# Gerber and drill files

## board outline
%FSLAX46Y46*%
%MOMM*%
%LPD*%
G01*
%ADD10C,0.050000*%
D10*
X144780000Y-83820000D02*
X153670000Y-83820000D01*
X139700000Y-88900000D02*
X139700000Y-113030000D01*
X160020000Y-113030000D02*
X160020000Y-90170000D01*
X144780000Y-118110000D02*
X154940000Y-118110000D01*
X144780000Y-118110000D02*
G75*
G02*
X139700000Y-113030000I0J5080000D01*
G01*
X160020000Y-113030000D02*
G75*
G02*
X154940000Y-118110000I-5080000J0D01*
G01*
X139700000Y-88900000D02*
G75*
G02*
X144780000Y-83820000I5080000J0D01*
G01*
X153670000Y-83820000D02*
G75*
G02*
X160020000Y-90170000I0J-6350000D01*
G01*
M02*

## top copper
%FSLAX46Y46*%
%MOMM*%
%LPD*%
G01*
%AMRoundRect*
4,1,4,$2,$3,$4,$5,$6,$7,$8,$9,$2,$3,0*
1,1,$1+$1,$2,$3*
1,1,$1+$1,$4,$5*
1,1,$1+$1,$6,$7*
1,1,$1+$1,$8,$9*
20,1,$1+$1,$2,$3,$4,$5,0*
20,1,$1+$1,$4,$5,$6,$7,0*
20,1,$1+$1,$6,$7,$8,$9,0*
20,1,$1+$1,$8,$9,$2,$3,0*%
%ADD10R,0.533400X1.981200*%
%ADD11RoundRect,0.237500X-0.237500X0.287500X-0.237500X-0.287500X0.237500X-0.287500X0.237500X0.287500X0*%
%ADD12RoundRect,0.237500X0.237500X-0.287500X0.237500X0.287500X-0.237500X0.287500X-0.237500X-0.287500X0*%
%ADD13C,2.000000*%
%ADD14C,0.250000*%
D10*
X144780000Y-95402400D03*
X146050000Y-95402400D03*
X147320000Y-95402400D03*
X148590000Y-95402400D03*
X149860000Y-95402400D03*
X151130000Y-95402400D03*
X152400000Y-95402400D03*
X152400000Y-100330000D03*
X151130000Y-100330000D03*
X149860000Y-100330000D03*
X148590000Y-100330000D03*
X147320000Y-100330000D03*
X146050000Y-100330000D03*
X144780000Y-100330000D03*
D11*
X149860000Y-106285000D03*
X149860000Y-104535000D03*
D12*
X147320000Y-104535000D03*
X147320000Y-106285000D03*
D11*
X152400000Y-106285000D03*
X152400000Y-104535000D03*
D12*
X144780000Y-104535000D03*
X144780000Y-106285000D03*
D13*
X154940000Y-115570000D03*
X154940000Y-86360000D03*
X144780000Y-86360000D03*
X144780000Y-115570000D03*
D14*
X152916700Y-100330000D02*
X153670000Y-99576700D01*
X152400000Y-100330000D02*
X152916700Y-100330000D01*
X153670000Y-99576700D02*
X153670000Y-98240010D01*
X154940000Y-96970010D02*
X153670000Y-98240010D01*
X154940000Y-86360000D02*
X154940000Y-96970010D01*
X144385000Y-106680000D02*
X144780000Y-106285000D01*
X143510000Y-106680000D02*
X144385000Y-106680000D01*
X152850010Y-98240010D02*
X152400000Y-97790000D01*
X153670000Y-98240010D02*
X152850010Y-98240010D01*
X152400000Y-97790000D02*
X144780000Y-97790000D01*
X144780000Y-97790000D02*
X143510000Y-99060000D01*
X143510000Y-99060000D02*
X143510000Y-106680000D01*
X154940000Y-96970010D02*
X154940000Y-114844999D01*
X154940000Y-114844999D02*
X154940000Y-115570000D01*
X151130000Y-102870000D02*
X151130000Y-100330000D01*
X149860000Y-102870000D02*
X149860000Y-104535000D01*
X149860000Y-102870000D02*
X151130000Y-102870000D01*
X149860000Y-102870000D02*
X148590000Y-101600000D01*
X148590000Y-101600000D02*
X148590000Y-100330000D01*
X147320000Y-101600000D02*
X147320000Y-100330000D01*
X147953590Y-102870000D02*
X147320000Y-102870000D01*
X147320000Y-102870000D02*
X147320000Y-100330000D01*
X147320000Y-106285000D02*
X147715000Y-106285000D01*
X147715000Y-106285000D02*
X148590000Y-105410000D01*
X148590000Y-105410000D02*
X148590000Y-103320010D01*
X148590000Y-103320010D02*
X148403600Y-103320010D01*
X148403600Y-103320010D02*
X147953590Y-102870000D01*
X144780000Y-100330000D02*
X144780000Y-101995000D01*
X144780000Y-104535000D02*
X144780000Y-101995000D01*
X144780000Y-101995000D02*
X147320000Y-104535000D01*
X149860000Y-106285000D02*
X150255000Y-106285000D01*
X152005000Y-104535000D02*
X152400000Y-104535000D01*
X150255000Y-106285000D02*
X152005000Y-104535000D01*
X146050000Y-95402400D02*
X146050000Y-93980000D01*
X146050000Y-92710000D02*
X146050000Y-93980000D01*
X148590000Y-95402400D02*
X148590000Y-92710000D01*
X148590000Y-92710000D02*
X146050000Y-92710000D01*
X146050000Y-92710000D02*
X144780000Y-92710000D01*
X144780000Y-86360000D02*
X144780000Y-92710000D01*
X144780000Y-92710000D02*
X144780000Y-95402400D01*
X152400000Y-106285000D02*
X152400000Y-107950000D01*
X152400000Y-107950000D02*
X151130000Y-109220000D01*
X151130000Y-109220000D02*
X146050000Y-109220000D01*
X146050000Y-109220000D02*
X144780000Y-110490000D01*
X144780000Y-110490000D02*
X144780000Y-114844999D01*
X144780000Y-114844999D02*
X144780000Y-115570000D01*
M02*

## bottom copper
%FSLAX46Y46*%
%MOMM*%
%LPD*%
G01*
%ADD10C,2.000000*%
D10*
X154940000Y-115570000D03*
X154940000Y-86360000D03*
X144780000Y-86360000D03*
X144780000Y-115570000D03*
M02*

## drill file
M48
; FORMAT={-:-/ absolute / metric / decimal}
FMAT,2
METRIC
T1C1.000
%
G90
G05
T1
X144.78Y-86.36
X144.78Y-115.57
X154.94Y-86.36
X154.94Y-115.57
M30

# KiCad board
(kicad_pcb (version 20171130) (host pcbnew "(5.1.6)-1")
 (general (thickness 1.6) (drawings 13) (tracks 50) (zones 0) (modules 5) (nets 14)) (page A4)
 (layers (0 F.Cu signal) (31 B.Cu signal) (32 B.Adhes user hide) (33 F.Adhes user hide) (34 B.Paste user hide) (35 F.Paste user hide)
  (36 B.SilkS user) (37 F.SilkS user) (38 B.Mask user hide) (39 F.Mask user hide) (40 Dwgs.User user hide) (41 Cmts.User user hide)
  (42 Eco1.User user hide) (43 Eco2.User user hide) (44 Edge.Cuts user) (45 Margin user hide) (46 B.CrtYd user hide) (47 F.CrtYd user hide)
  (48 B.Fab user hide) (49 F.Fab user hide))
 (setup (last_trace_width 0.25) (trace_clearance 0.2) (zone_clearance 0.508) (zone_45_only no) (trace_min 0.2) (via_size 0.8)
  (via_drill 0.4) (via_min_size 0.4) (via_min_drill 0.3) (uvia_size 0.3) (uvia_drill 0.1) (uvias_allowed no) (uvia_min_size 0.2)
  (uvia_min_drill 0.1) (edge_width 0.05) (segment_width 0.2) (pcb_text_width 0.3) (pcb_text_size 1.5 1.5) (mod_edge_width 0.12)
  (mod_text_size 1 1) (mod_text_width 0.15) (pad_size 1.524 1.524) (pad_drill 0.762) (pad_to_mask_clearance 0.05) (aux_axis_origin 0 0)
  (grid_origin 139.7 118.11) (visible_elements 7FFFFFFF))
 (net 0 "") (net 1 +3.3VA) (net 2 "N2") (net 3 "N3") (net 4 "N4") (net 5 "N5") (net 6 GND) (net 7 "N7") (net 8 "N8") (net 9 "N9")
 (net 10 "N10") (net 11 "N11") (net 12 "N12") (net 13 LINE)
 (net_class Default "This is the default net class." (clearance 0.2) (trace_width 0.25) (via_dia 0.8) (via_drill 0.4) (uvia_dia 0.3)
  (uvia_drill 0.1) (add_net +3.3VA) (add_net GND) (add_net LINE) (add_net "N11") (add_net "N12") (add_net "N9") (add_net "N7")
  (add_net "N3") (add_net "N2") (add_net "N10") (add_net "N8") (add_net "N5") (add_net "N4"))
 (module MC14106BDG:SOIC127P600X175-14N (layer F.Cu) (at 148.59 97.8662 90)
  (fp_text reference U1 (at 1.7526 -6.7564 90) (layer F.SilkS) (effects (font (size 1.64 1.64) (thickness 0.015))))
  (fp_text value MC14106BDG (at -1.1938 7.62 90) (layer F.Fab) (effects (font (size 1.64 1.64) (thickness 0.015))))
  (pad 14 smd rect (at 2.4638 -3.81 90) (size 1.9812 0.5334) (layers F.Cu F.Paste F.Mask) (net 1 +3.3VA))
  (pad 13 smd rect (at 2.4638 -2.54 90) (size 1.9812 0.5334) (layers F.Cu F.Paste F.Mask) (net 1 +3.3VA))
  (pad 12 smd rect (at 2.4638 -1.27 90) (size 1.9812 0.5334) (layers F.Cu F.Paste F.Mask) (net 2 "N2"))
  (pad 11 smd rect (at 2.4638 0 90) (size 1.9812 0.5334) (layers F.Cu F.Paste F.Mask) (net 1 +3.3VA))
  (pad 10 smd rect (at 2.4638 1.27 90) (size 1.9812 0.5334) (layers F.Cu F.Paste F.Mask) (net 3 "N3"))
  (pad 9 smd rect (at 2.4638 2.54 90) (size 1.9812 0.5334) (layers F.Cu F.Paste F.Mask) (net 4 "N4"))
  (pad 8 smd rect (at 2.4638 3.81 90) (size 1.9812 0.5334) (layers F.Cu F.Paste F.Mask) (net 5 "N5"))
  (pad 7 smd rect (at -2.4638 3.81 90) (size 1.9812 0.5334) (layers F.Cu F.Paste F.Mask) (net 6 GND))
  (pad 6 smd rect (at -2.4638 2.54 90) (size 1.9812 0.5334) (layers F.Cu F.Paste F.Mask) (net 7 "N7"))
  (pad 5 smd rect (at -2.4638 1.27 90) (size 1.9812 0.5334) (layers F.Cu F.Paste F.Mask) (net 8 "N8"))
  (pad 4 smd rect (at -2.4638 0 90) (size 1.9812 0.5334) (layers F.Cu F.Paste F.Mask) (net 7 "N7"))
  (pad 3 smd rect (at -2.4638 -1.27 90) (size 1.9812 0.5334) (layers F.Cu F.Paste F.Mask) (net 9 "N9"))
  (pad 2 smd rect (at -2.4638 -2.54 90) (size 1.9812 0.5334) (layers F.Cu F.Paste F.Mask) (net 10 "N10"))
  (pad 1 smd rect (at -2.4638 -3.81 90) (size 1.9812 0.5334) (layers F.Cu F.Paste F.Mask) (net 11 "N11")))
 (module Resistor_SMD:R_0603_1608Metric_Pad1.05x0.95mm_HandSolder (layer F.Cu) (at 149.86 105.41 270)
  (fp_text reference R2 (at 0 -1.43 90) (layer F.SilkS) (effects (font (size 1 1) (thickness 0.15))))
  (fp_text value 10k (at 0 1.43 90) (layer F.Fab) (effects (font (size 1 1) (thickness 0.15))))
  (pad 2 smd roundrect (at 0.875 0 270) (size 1.05 0.95) (layers F.Cu F.Paste F.Mask) (roundrect_rratio 0.25) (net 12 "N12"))
  (pad 1 smd roundrect (at -0.875 0 270) (size 1.05 0.95) (layers F.Cu F.Paste F.Mask) (roundrect_rratio 0.25) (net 7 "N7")))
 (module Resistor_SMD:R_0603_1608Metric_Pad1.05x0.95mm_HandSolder (layer F.Cu) (at 147.32 105.41 90)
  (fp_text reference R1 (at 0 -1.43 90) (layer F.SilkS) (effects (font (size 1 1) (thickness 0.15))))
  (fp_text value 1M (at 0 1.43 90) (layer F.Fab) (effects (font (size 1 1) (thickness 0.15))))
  (pad 2 smd roundrect (at 0.875 0 90) (size 1.05 0.95) (layers F.Cu F.Paste F.Mask) (roundrect_rratio 0.25) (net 11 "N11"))
  (pad 1 smd roundrect (at -0.875 0 90) (size 1.05 0.95) (layers F.Cu F.Paste F.Mask) (roundrect_rratio 0.25) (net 9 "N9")))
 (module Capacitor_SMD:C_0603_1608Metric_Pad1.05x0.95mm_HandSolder (layer F.Cu) (at 152.4 105.41 270)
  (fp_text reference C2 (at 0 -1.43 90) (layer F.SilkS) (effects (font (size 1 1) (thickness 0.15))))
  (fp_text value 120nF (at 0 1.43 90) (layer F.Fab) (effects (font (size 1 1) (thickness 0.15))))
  (pad 2 smd roundrect (at 0.875 0 270) (size 1.05 0.95) (layers F.Cu F.Paste F.Mask) (roundrect_rratio 0.25) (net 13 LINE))
  (pad 1 smd roundrect (at -0.875 0 270) (size 1.05 0.95) (layers F.Cu F.Paste F.Mask) (roundrect_rratio 0.25) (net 12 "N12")))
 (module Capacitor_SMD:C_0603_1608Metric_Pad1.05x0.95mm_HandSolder (layer F.Cu) (at 144.78 105.41 90)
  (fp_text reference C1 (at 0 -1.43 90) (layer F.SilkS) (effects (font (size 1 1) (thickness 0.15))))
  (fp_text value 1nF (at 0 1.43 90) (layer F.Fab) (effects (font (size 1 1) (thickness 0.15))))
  (pad 2 smd roundrect (at 0.875 0 90) (size 1.05 0.95) (layers F.Cu F.Paste F.Mask) (roundrect_rratio 0.25) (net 11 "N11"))
  (pad 1 smd roundrect (at -0.875 0 90) (size 1.05 0.95) (layers F.Cu F.Paste F.Mask) (roundrect_rratio 0.25) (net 6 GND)))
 (gr_line (start 144.78 83.82) (end 153.67 83.82) (layer Edge.Cuts) (width 0.05))
 (gr_line (start 139.7 88.9) (end 139.7 113.03) (layer Edge.Cuts) (width 0.05))
 (gr_line (start 160.02 113.03) (end 160.02 90.17) (layer Edge.Cuts) (width 0.05))
 (gr_line (start 144.78 118.11) (end 154.94 118.11) (layer Edge.Cuts) (width 0.05))
 (gr_arc (start 144.78 113.03) (end 139.7 113.03) (angle -90) (layer Edge.Cuts) (width 0.05))
 (gr_arc (start 154.94 113.03) (end 154.94 118.11) (angle -90) (layer Edge.Cuts) (width 0.05))
 (gr_arc (start 144.78 88.9) (end 144.78 83.82) (angle -90) (layer Edge.Cuts) (width 0.05))
 (gr_arc (start 153.67 90.17) (end 160.02 90.17) (angle -90) (layer Edge.Cuts) (width 0.05))
 (via (at 154.94 115.57) (size 2) (drill 1) (layers F.Cu B.Cu) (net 6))
 (via (at 154.94 86.36) (size 2) (drill 1) (layers F.Cu B.Cu) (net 6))
 (segment (start 152.9167 100.33) (end 153.67 99.5767) (width 0.25) (layer F.Cu) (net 6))
 (segment (start 152.4 100.33) (end 152.9167 100.33) (width 0.25) (layer F.Cu) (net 6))
 (segment (start 153.67 99.5767) (end 153.67 98.24001) (width 0.25) (layer F.Cu) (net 6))
 (segment (start 154.94 96.97001) (end 153.67 98.24001) (width 0.25) (layer F.Cu) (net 6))
 (segment (start 154.94 86.36) (end 154.94 96.97001) (width 0.25) (layer F.Cu) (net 6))
 (segment (start 144.385 106.68) (end 144.78 106.285) (width 0.25) (layer F.Cu) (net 6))
 (segment (start 143.51 106.68) (end 144.385 106.68) (width 0.25) (layer F.Cu) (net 6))
 (segment (start 152.85001 98.24001) (end 152.4 97.79) (width 0.25) (layer F.Cu) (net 6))
 (segment (start 153.67 98.24001) (end 152.85001 98.24001) (width 0.25) (layer F.Cu) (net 6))
 (segment (start 152.4 97.79) (end 144.78 97.79) (width 0.25) (layer F.Cu) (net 6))
 (segment (start 144.78 97.79) (end 143.51 99.06) (width 0.25) (layer F.Cu) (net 6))
 (segment (start 143.51 99.06) (end 143.51 106.68) (width 0.25) (layer F.Cu) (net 6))
 (segment (start 154.94 96.97001) (end 154.94 114.844999) (width 0.25) (layer F.Cu) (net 6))
 (segment (start 154.94 114.844999) (end 154.94 115.57) (width 0.25) (layer F.Cu) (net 6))
 (segment (start 151.13 102.87) (end 151.13 100.33) (width 0.25) (layer F.Cu) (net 7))
 (segment (start 149.86 102.87) (end 149.86 104.535) (width 0.25) (layer F.Cu) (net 7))
 (segment (start 149.86 102.87) (end 151.13 102.87) (width 0.25) (layer F.Cu) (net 7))
 (segment (start 149.86 102.87) (end 148.59 101.6) (width 0.25) (layer F.Cu) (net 7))
 (segment (start 148.59 101.6) (end 148.59 100.33) (width 0.25) (layer F.Cu) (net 7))
 (segment (start 147.32 101.6) (end 147.32 100.33) (width 0.25) (layer F.Cu) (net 9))
 (segment (start 147.95359 102.87) (end 147.32 102.87) (width 0.25) (layer F.Cu) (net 9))
 (segment (start 147.32 102.87) (end 147.32 100.33) (width 0.25) (layer F.Cu) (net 9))
 (segment (start 147.32 106.285) (end 147.715 106.285) (width 0.25) (layer F.Cu) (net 9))
 (segment (start 147.715 106.285) (end 148.59 105.41) (width 0.25) (layer F.Cu) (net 9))
 (segment (start 148.59 105.41) (end 148.59 103.32001) (width 0.25) (layer F.Cu) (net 9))
 (segment (start 148.59 103.32001) (end 148.4036 103.32001) (width 0.25) (layer F.Cu) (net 9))
 (segment (start 148.4036 103.32001) (end 147.95359 102.87) (width 0.25) (layer F.Cu) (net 9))
 (segment (start 144.78 100.33) (end 144.78 101.995) (width 0.25) (layer F.Cu) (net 11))
 (segment (start 144.78 104.535) (end 144.78 101.995) (width 0.25) (layer F.Cu) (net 11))
 (segment (start 144.78 101.995) (end 147.32 104.535) (width 0.25) (layer F.Cu) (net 11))
 (segment (start 149.86 106.285) (end 150.255 106.285) (width 0.25) (layer F.Cu) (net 12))
 (segment (start 152.005 104.535) (end 152.4 104.535) (width 0.25) (layer F.Cu) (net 12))
 (segment (start 150.255 106.285) (end 152.005 104.535) (width 0.25) (layer F.Cu) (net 12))
 (via (at 144.78 86.36) (size 2) (drill 1) (layers F.Cu B.Cu) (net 1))
 (segment (start 146.05 95.4024) (end 146.05 93.98) (width 0.25) (layer F.Cu) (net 1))
 (segment (start 146.05 92.71) (end 146.05 93.98) (width 0.25) (layer F.Cu) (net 1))
 (segment (start 148.59 95.4024) (end 148.59 92.71) (width 0.25) (layer F.Cu) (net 1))
 (segment (start 148.59 92.71) (end 146.05 92.71) (width 0.25) (layer F.Cu) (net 1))
 (segment (start 146.05 92.71) (end 144.78 92.71) (width 0.25) (layer F.Cu) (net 1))
 (segment (start 144.78 86.36) (end 144.78 92.71) (width 0.25) (layer F.Cu) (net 1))
 (segment (start 144.78 92.71) (end 144.78 95.4024) (width 0.25) (layer F.Cu) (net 1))
 (via (at 144.78 115.57) (size 2) (drill 1) (layers F.Cu B.Cu) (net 13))
 (segment (start 152.4 106.285) (end 152.4 107.95) (width 0.25) (layer F.Cu) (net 13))
 (segment (start 152.4 107.95) (end 151.13 109.22) (width 0.25) (layer F.Cu) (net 13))
 (segment (start 151.13 109.22) (end 146.05 109.22) (width 0.25) (layer F.Cu) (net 13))
 (segment (start 146.05 109.22) (end 144.78 110.49) (width 0.25) (layer F.Cu) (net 13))
 (segment (start 144.78 110.49) (end 144.78 114.844999) (width 0.25) (layer F.Cu) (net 13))
 (segment (start 144.78 114.844999) (end 144.78 115.57) (width 0.25) (layer F.Cu) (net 13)))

